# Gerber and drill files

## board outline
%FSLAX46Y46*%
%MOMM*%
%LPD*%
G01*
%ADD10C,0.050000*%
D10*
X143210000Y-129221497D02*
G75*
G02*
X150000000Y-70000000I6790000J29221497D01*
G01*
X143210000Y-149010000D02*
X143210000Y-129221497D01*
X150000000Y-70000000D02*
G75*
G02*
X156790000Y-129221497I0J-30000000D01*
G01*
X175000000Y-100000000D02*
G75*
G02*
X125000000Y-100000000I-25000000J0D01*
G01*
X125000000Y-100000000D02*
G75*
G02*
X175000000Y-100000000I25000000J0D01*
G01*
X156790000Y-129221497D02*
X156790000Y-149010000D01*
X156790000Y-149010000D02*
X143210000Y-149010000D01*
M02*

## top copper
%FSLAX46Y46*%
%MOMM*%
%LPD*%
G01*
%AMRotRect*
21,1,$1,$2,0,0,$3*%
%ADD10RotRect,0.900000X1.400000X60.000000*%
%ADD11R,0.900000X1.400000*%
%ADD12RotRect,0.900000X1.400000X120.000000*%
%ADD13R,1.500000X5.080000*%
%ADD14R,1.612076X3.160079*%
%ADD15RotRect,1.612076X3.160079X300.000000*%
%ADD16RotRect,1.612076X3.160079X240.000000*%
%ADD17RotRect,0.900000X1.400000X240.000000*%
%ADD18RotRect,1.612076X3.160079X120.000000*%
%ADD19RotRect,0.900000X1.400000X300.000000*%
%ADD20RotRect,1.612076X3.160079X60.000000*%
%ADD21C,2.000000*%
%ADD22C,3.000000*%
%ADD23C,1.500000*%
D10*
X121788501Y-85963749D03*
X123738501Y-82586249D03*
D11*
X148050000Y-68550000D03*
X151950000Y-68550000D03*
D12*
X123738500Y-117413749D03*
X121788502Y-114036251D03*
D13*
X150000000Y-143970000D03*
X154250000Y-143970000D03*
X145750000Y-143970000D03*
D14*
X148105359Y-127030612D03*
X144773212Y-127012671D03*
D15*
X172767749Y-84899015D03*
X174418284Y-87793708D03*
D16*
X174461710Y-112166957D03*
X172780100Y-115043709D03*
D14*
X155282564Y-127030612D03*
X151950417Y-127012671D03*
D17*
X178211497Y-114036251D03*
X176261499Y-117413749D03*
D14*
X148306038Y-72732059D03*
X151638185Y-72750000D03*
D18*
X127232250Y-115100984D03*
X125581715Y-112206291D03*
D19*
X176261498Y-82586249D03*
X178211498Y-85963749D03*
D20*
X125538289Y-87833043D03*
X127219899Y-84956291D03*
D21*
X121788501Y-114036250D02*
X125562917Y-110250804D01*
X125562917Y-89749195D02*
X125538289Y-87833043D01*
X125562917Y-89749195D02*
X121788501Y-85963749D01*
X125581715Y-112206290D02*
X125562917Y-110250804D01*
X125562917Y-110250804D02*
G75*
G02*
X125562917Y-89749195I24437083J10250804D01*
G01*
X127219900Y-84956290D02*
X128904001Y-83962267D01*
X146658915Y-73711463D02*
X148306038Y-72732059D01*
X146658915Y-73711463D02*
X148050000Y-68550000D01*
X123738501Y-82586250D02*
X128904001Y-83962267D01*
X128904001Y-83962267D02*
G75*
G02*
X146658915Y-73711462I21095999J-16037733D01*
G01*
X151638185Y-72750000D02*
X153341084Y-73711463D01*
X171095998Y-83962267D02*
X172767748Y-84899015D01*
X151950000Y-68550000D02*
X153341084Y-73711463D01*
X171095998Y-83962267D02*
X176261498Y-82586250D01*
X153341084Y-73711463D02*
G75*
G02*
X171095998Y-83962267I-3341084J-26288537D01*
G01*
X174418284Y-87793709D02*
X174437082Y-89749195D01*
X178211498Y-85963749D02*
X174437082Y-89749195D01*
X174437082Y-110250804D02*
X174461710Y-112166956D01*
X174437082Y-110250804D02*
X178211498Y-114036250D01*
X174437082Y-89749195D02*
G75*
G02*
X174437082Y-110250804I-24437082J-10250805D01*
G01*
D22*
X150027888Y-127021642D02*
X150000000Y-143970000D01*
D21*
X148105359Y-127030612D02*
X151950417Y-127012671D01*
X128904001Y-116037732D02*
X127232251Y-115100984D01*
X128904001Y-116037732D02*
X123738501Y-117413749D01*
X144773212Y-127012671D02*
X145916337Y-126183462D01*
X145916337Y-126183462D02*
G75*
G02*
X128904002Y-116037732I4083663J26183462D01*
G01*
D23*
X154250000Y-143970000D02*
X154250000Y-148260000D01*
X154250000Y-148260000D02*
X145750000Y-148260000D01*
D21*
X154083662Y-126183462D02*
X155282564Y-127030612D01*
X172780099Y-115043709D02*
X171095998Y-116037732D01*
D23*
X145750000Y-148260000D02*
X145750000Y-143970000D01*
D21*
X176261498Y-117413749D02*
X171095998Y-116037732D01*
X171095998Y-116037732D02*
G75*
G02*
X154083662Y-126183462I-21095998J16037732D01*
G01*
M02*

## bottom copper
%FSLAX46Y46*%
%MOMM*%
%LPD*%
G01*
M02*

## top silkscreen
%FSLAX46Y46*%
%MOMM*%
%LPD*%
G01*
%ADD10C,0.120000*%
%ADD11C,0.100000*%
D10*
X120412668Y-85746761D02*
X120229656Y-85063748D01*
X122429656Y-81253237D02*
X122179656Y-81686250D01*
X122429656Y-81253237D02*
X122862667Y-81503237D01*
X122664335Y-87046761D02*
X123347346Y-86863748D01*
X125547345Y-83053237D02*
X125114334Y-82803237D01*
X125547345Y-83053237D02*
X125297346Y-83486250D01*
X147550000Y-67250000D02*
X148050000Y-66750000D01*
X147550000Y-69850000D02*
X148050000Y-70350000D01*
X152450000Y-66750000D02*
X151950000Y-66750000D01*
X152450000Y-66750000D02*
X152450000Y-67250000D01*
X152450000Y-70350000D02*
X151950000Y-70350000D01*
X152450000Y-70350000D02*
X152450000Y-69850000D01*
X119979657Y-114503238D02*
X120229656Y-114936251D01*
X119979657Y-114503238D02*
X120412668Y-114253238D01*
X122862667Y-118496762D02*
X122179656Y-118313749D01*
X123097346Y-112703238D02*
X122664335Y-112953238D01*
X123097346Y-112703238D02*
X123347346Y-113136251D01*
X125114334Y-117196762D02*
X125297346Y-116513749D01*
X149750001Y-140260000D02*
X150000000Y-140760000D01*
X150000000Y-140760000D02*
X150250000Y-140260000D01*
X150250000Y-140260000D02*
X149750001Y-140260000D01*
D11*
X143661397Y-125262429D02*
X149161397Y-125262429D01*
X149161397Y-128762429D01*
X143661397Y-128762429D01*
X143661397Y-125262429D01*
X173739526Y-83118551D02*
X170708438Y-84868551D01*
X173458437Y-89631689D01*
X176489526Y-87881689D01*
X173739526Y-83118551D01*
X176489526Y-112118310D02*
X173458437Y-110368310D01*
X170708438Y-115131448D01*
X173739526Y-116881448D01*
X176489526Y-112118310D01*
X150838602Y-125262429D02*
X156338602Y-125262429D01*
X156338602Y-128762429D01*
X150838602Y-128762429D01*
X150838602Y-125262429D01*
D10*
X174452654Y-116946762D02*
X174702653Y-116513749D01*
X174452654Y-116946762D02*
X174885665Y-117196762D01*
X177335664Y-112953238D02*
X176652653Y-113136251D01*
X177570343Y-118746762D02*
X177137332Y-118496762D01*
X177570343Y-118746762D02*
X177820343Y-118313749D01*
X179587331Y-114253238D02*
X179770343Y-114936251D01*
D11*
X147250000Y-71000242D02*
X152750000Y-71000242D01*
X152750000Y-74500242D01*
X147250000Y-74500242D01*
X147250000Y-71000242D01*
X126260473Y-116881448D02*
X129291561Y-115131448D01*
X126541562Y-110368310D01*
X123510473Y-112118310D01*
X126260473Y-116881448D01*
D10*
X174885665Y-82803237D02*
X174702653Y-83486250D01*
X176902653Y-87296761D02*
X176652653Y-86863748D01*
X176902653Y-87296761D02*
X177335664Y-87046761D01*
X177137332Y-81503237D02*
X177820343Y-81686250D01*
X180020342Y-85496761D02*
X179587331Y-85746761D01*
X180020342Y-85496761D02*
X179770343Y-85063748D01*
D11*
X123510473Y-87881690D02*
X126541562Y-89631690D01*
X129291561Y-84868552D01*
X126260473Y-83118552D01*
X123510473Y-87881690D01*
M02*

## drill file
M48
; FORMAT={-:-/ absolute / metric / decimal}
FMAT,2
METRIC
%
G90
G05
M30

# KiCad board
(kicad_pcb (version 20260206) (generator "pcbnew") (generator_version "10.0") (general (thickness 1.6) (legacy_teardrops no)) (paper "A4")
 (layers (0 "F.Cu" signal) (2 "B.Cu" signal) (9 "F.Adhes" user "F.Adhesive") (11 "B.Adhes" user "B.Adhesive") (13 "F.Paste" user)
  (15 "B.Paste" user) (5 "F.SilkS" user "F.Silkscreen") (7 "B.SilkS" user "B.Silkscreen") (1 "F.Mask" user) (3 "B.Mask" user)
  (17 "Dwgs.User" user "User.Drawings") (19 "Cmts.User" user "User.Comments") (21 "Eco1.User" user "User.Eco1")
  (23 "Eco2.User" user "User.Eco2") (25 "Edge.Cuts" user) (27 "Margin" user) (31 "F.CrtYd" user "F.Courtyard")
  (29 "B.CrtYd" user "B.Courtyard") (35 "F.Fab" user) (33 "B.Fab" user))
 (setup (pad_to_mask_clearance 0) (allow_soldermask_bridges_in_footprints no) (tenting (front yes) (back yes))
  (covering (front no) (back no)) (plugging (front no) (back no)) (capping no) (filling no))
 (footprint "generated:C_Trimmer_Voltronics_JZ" (layer "F.Cu") (at 122.763501 84.274999 60)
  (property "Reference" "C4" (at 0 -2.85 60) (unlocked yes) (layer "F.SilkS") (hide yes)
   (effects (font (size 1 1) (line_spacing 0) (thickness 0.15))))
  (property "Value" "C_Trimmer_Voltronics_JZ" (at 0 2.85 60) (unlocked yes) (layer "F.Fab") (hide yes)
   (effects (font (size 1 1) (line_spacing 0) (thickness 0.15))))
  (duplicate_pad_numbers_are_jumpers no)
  (fp_line (start -2.45 -1.3) (end -1.949999 -1.8) (stroke (width 0.12) (type default)) (layer "F.SilkS"))
  (fp_line (start 2.45 -1.799999) (end 1.95 -1.799999) (stroke (width 0.12) (type default)) (layer "F.SilkS"))
  (fp_line (start 2.45 -1.799999) (end 2.449999 -1.300001) (stroke (width 0.12) (type default)) (layer "F.SilkS"))
  (fp_line (start -2.449999 1.300001) (end -1.95 1.799999) (stroke (width 0.12) (type default)) (layer "F.SilkS"))
  (fp_line (start 2.449999 1.799999) (end 2.45 1.3) (stroke (width 0.12) (type default)) (layer "F.SilkS"))
  (fp_line (start 2.449999 1.799999) (end 1.949999 1.8) (stroke (width 0.12) (type default)) (layer "F.SilkS"))
  (pad "1" smd rect (at -1.95 0 60) (size 0.9 1.4) (layers "F.Cu" "F.Mask" "F.Paste") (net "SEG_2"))
  (pad "2" smd rect (at 1.95 0 60) (size 0.9 1.4) (layers "F.Cu" "F.Mask" "F.Paste") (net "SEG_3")))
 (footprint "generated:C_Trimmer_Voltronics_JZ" (layer "F.Cu") (at 150 68.55)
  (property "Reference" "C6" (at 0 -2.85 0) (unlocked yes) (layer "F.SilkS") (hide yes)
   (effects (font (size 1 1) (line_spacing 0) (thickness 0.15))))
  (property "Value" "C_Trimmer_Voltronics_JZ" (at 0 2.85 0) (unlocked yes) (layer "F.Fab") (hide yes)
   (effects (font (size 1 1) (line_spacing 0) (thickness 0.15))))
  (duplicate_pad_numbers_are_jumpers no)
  (fp_line (start -2.45 -1.3) (end -1.95 -1.8) (stroke (width 0.12) (type default)) (layer "F.SilkS"))
  (fp_line (start -2.45 1.3) (end -1.95 1.8) (stroke (width 0.12) (type default)) (layer "F.SilkS"))
  (fp_line (start 2.45 -1.8) (end 1.95 -1.8) (stroke (width 0.12) (type default)) (layer "F.SilkS"))
  (fp_line (start 2.45 -1.8) (end 2.45 -1.3) (stroke (width 0.12) (type default)) (layer "F.SilkS"))
  (fp_line (start 2.45 1.8) (end 1.95 1.8) (stroke (width 0.12) (type default)) (layer "F.SilkS"))
  (fp_line (start 2.45 1.8) (end 2.45 1.3) (stroke (width 0.12) (type default)) (layer "F.SilkS"))
  (pad "1" smd rect (at -1.95 0) (size 0.9 1.4) (layers "F.Cu" "F.Mask" "F.Paste") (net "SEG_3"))
  (pad "2" smd rect (at 1.95 0) (size 0.9 1.4) (layers "F.Cu" "F.Mask" "F.Paste") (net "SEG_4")))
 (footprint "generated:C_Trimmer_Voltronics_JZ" (layer "F.Cu") (at 122.763501 115.725 120)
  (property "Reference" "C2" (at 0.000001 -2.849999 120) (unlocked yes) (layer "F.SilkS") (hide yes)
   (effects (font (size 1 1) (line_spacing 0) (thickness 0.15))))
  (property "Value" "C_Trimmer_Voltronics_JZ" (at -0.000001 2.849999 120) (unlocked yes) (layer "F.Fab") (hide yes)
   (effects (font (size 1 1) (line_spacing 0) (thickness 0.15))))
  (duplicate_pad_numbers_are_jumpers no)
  (fp_line (start 2.449999 -1.799999) (end 1.949999 -1.8) (stroke (width 0.12) (type default)) (layer "F.SilkS"))
  (fp_line (start 2.449999 -1.799999) (end 2.45 -1.3) (stroke (width 0.12) (type default)) (layer "F.SilkS"))
  (fp_line (start -2.449999 -1.300001) (end -1.95 -1.799999) (stroke (width 0.12) (type default)) (layer "F.SilkS"))
  (fp_line (start 2.45 1.799999) (end 2.449999 1.300001) (stroke (width 0.12) (type default)) (layer "F.SilkS"))
  (fp_line (start 2.45 1.799999) (end 1.95 1.799999) (stroke (width 0.12) (type default)) (layer "F.SilkS"))
  (fp_line (start -2.45 1.3) (end -1.949999 1.8) (stroke (width 0.12) (type default)) (layer "F.SilkS"))
  (pad "1" smd rect (at -1.949999 -0.000001 120) (size 0.9 1.4) (layers "F.Cu" "F.Mask" "F.Paste") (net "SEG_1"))
  (pad "2" smd rect (at 1.949999 0.000001 120) (size 0.9 1.4) (layers "F.Cu" "F.Mask" "F.Paste") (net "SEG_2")))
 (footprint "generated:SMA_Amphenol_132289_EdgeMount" (layer "F.Cu") (at 150 143.97 -90)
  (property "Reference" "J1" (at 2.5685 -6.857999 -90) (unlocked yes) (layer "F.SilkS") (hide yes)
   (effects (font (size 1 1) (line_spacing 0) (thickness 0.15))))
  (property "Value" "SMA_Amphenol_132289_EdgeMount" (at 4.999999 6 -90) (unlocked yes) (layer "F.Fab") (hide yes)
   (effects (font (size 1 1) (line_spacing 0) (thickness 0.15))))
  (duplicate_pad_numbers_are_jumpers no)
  (fp_line (start -3.71 0.249999) (end -3.21 0) (stroke (width 0.12) (type default)) (layer "F.SilkS"))
  (fp_line (start -3.21 0) (end -3.71 -0.25) (stroke (width 0.12) (type default)) (layer "F.SilkS"))
  (fp_line (start -3.71 -0.25) (end -3.71 0.249999) (stroke (width 0.12) (type default)) (layer "F.SilkS"))
  (pad "1" smd rect (at 0 0) (size 1.5 5.08) (layers "F.Cu" "F.Mask" "F.Paste") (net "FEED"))
  (pad "2" smd rect (at 0 -4.25) (size 1.5 5.08) (layers "F.Cu" "F.Mask" "F.Paste") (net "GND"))
  (pad "2" smd rect (at 0 4.25) (size 1.5 5.08) (layers "F.Cu" "F.Mask" "F.Paste") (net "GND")))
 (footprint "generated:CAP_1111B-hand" (layer "F.Cu") (at 146.411397 127.012671 180)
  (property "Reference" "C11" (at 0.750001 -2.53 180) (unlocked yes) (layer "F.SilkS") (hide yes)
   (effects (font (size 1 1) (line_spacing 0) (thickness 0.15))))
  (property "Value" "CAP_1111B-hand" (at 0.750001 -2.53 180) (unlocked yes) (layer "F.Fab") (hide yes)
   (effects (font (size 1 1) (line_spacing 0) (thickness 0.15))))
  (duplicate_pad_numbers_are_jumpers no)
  (fp_rect (start -2.75 -1.749758) (end 2.75 1.750242) (stroke (width 0.1) (type default)) (fill no) (layer "F.SilkS"))
  (pad "1" smd rect (at -1.693962 -0.017941 180) (size 1.612076 3.160079) (layers "F.Cu" "F.Mask" "F.Paste") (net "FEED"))
  (pad "2" smd rect (at 1.638185 0 180) (size 1.612076 3.160079) (layers "F.Cu" "F.Mask" "F.Paste") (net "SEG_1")))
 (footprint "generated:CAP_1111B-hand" (layer "F.Cu") (at 173.599192 86.374999 -60)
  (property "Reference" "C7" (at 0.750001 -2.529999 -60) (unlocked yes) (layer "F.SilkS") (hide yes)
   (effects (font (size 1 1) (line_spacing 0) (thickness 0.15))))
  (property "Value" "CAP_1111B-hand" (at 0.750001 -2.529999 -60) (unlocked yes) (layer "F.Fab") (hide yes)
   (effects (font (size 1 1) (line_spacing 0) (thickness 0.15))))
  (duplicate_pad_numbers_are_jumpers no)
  (fp_poly
   (pts (xy -2.75 -1.749757) (xy -2.749999 1.750242) (xy 2.749999 1.750242) (xy 2.749999 -1.749758)) (stroke (width 0.1) (type default))
   (fill no) (layer "F.SilkS"))
  (pad "1" smd rect (at -1.693961 -0.017941 -60) (size 1.612076 3.160079) (layers "F.Cu" "F.Mask" "F.Paste") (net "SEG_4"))
  (pad "2" smd rect (at 1.638184 0 -60) (size 1.612076 3.160079) (layers "F.Cu" "F.Mask" "F.Paste") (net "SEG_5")))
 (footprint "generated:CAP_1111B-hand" (layer "F.Cu") (at 173.599192 113.625 -120)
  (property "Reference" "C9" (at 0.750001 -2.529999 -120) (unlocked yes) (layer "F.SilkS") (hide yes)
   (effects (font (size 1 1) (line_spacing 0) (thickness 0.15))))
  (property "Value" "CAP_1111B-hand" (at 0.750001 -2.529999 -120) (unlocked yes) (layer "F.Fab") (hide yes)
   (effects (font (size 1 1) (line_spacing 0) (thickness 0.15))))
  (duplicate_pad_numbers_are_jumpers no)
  (fp_poly
   (pts (xy -2.749999 -1.749758) (xy -2.749999 1.750242) (xy 2.749999 1.750242) (xy 2.75 -1.749757)) (stroke (width 0.1) (type default))
   (fill no) (layer "F.SilkS"))
  (pad "1" smd rect (at -1.693961 -0.017941 -120) (size 1.612076 3.160079) (layers "F.Cu" "F.Mask" "F.Paste") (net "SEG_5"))
  (pad "2" smd rect (at 1.638184 0 -120) (size 1.612076 3.160079) (layers "F.Cu" "F.Mask" "F.Paste") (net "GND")))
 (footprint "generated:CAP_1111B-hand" (layer "F.Cu") (at 153.588602 127.012671 180)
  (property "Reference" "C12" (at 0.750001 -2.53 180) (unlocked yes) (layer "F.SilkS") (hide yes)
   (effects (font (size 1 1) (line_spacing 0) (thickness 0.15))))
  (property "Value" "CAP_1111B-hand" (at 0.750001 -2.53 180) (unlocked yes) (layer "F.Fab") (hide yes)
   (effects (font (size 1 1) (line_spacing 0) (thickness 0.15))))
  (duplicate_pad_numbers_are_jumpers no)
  (fp_rect (start -2.75 -1.749758) (end 2.75 1.750242) (stroke (width 0.1) (type default)) (fill no) (layer "F.SilkS"))
  (pad "1" smd rect (at -1.693962 -0.017941 180) (size 1.612076 3.160079) (layers "F.Cu" "F.Mask" "F.Paste") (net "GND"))
  (pad "2" smd rect (at 1.638185 0 180) (size 1.612076 3.160079) (layers "F.Cu" "F.Mask" "F.Paste") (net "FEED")))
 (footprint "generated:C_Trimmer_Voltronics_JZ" (layer "F.Cu") (at 177.236498 115.725 -120)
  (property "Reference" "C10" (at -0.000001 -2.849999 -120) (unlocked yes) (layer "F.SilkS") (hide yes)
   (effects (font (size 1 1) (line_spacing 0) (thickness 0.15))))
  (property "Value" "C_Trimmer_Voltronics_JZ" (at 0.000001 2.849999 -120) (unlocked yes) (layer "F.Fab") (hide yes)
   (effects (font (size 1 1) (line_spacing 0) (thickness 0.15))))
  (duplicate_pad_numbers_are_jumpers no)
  (fp_line (start 2.449999 1.799999) (end 1.949999 1.8) (stroke (width 0.12) (type default)) (layer "F.SilkS"))
  (fp_line (start 2.449999 1.799999) (end 2.45 1.3) (stroke (width 0.12) (type default)) (layer "F.SilkS"))
  (fp_line (start -2.449999 1.300001) (end -1.95 1.799999) (stroke (width 0.12) (type default)) (layer "F.SilkS"))
  (fp_line (start 2.45 -1.799999) (end 2.449999 -1.300001) (stroke (width 0.12) (type default)) (layer "F.SilkS"))
  (fp_line (start 2.45 -1.799999) (end 1.95 -1.799999) (stroke (width 0.12) (type default)) (layer "F.SilkS"))
  (fp_line (start -2.45 -1.3) (end -1.949999 -1.8) (stroke (width 0.12) (type default)) (layer "F.SilkS"))
  (pad "1" smd rect (at -1.949999 0.000001 -120) (size 0.9 1.4) (layers "F.Cu" "F.Mask" "F.Paste") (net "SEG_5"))
  (pad "2" smd rect (at 1.949999 -0.000001 -120) (size 0.9 1.4) (layers "F.Cu" "F.Mask" "F.Paste") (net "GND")))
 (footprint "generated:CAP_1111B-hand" (layer "F.Cu") (at 150 72.75)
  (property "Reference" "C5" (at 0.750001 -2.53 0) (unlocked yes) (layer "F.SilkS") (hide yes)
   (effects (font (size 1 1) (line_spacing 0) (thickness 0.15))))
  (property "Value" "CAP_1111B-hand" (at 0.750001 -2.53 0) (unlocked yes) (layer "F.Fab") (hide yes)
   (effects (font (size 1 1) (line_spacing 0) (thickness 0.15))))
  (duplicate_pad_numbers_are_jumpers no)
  (fp_rect (start -2.75 -1.749758) (end 2.75 1.750242) (stroke (width 0.1) (type default)) (fill no) (layer "F.SilkS"))
  (pad "1" smd rect (at -1.693962 -0.017941) (size 1.612076 3.160079) (layers "F.Cu" "F.Mask" "F.Paste") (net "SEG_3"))
  (pad "2" smd rect (at 1.638185 0) (size 1.612076 3.160079) (layers "F.Cu" "F.Mask" "F.Paste") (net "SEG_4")))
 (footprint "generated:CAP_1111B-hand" (layer "F.Cu") (at 126.400807 113.625 120)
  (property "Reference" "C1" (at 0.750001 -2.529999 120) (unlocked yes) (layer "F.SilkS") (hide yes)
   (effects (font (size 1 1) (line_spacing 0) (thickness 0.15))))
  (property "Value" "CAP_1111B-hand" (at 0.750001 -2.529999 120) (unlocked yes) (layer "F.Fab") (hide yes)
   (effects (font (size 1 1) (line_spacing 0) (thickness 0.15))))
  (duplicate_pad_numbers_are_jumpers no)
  (fp_poly
   (pts (xy -2.75 -1.749757) (xy -2.749999 1.750242) (xy 2.749999 1.750242) (xy 2.749999 -1.749758)) (stroke (width 0.1) (type default))
   (fill no) (layer "F.SilkS"))
  (pad "1" smd rect (at -1.693961 -0.017941 120) (size 1.612076 3.160079) (layers "F.Cu" "F.Mask" "F.Paste") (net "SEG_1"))
  (pad "2" smd rect (at 1.638184 0 120) (size 1.612076 3.160079) (layers "F.Cu" "F.Mask" "F.Paste") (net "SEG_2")))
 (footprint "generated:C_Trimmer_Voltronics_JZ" (layer "F.Cu") (at 177.236498 84.274999 -60)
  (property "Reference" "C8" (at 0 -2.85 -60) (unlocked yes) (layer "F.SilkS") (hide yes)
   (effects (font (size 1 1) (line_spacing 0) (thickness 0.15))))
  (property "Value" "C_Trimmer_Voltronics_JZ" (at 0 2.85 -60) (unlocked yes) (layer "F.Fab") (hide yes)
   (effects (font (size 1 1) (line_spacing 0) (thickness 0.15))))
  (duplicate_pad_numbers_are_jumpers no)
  (fp_line (start -2.45 1.3) (end -1.949999 1.8) (stroke (width 0.12) (type default)) (layer "F.SilkS"))
  (fp_line (start 2.45 1.799999) (end 1.95 1.799999) (stroke (width 0.12) (type default)) (layer "F.SilkS"))
  (fp_line (start 2.45 1.799999) (end 2.449999 1.300001) (stroke (width 0.12) (type default)) (layer "F.SilkS"))
  (fp_line (start -2.449999 -1.300001) (end -1.95 -1.799999) (stroke (width 0.12) (type default)) (layer "F.SilkS"))
  (fp_line (start 2.449999 -1.799999) (end 2.45 -1.3) (stroke (width 0.12) (type default)) (layer "F.SilkS"))
  (fp_line (start 2.449999 -1.799999) (end 1.949999 -1.8) (stroke (width 0.12) (type default)) (layer "F.SilkS"))
  (pad "1" smd rect (at -1.95 0 -60) (size 0.9 1.4) (layers "F.Cu" "F.Mask" "F.Paste") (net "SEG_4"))
  (pad "2" smd rect (at 1.95 0 -60) (size 0.9 1.4) (layers "F.Cu" "F.Mask" "F.Paste") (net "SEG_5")))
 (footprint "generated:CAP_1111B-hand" (layer "F.Cu") (at 126.400807 86.375 60)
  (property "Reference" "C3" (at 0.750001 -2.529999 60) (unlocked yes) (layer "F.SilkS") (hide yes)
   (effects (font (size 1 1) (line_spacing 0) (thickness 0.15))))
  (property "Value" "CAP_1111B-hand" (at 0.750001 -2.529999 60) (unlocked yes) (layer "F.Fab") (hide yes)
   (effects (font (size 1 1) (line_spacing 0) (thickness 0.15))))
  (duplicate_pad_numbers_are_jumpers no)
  (fp_poly
   (pts (xy -2.749999 -1.749758) (xy -2.749999 1.750242) (xy 2.749999 1.750242) (xy 2.75 -1.749757)) (stroke (width 0.1) (type default))
   (fill no) (layer "F.SilkS"))
  (pad "1" smd rect (at -1.693961 -0.017941 60) (size 1.612076 3.160079) (layers "F.Cu" "F.Mask" "F.Paste") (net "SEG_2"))
  (pad "2" smd rect (at 1.638184 0 60) (size 1.612076 3.160079) (layers "F.Cu" "F.Mask" "F.Paste") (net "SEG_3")))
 (gr_arc (start 143.21 129.221497) (mid 120.195261 96.582758) (end 150 70) (stroke (width 0.05) (type default)) (layer "Edge.Cuts"))
 (gr_line (start 143.21 149.01) (end 143.21 129.221497) (stroke (width 0.05) (type default)) (layer "Edge.Cuts"))
 (gr_arc (start 150 70) (mid 179.804738 96.582758) (end 156.79 129.221497) (stroke (width 0.05) (type default)) (layer "Edge.Cuts"))
 (gr_circle (center 150 100) (end 175 100) (stroke (width 0.05) (type default)) (fill no) (layer "Edge.Cuts"))
 (gr_line (start 156.79 129.221497) (end 156.79 149.01) (stroke (width 0.05) (type default)) (layer "Edge.Cuts"))
 (gr_line (start 156.79 149.01) (end 143.21 149.01) (stroke (width 0.05) (type default)) (layer "Edge.Cuts"))
 (segment (start 121.788501 114.03625) (end 125.562917 110.250804) (width 2) (layer "F.Cu") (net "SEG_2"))
 (segment (start 125.562917 89.749195) (end 125.538289 87.833043) (width 2) (layer "F.Cu") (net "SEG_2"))
 (segment (start 125.562917 89.749195) (end 121.788501 85.963749) (width 2) (layer "F.Cu") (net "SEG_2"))
 (segment (start 125.581715 112.20629) (end 125.562917 110.250804) (width 2) (layer "F.Cu") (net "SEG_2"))
 (arc (start 125.562917 110.250804) (mid 123.5 100) (end 125.562917 89.749195) (width 2) (layer "F.Cu") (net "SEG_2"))
 (segment (start 127.2199 84.95629) (end 128.904001 83.962267) (width 2) (layer "F.Cu") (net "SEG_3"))
 (segment (start 146.658915 73.711463) (end 148.306038 72.732059) (width 2) (layer "F.Cu") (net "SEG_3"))
 (segment (start 146.658915 73.711463) (end 148.05 68.55) (width 2) (layer "F.Cu") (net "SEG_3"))
 (segment (start 123.738501 82.58625) (end 128.904001 83.962267) (width 2) (layer "F.Cu") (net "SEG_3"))
 (arc (start 128.904001 83.962267) (mid 136.75 77.050326) (end 146.658915 73.711463) (width 2) (layer "F.Cu") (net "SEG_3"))
 (segment (start 151.638185 72.75) (end 153.341084 73.711463) (width 2) (layer "F.Cu") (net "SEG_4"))
 (segment (start 171.095998 83.962267) (end 172.767748 84.899015) (width 2) (layer "F.Cu") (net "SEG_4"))
 (segment (start 151.95 68.55) (end 153.341084 73.711463) (width 2) (layer "F.Cu") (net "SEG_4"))
 (segment (start 171.095998 83.962267) (end 176.261498 82.58625) (width 2) (layer "F.Cu") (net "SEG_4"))
 (arc (start 153.341084 73.711463) (mid 163.25 77.050326) (end 171.095998 83.962267) (width 2) (layer "F.Cu") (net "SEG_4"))
 (segment (start 174.418284 87.793709) (end 174.437082 89.749195) (width 2) (layer "F.Cu") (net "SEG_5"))
 (segment (start 178.211498 85.963749) (end 174.437082 89.749195) (width 2) (layer "F.Cu") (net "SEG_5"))
 (segment (start 174.437082 110.250804) (end 174.46171 112.166956) (width 2) (layer "F.Cu") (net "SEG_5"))
 (segment (start 174.437082 110.250804) (end 178.211498 114.03625) (width 2) (layer "F.Cu") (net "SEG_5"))
 (arc (start 174.437082 89.749195) (mid 176.5 100) (end 174.437082 110.250804) (width 2) (layer "F.Cu") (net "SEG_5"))
 (segment (start 150.027888 127.021642) (end 150 143.97) (width 3) (layer "F.Cu") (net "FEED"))
 (segment (start 148.105359 127.030612) (end 151.950417 127.012671) (width 2) (layer "F.Cu") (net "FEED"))
 (segment (start 128.904001 116.037732) (end 127.232251 115.100984) (width 2) (layer "F.Cu") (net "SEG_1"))
 (segment (start 128.904001 116.037732) (end 123.738501 117.413749) (width 2) (layer "F.Cu") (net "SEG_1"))
 (segment (start 144.773212 127.012671) (end 145.916337 126.183462) (width 2) (layer "F.Cu") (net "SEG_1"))
 (arc (start 145.916337 126.183462) (mid 136.426577 122.759881) (end 128.904001 116.037732) (width 2) (layer "F.Cu") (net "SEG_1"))
 (segment (start 154.25 143.97) (end 154.25 148.26) (width 1.5) (layer "F.Cu") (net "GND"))
 (segment (start 154.25 148.26) (end 145.75 148.26) (width 1.5) (layer "F.Cu") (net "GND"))
 (segment (start 154.083662 126.183462) (end 155.282564 127.030612) (width 2) (layer "F.Cu") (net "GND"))
 (segment (start 172.780099 115.043709) (end 171.095998 116.037732) (width 2) (layer "F.Cu") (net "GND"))
 (segment (start 145.75 148.26) (end 145.75 143.97) (width 1.5) (layer "F.Cu") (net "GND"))
 (segment (start 176.261498 117.413749) (end 171.095998 116.037732) (width 2) (layer "F.Cu") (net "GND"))
 (arc (start 171.095998 116.037732) (mid 163.573422 122.759881) (end 154.083662 126.183462) (width 2) (layer "F.Cu") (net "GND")))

